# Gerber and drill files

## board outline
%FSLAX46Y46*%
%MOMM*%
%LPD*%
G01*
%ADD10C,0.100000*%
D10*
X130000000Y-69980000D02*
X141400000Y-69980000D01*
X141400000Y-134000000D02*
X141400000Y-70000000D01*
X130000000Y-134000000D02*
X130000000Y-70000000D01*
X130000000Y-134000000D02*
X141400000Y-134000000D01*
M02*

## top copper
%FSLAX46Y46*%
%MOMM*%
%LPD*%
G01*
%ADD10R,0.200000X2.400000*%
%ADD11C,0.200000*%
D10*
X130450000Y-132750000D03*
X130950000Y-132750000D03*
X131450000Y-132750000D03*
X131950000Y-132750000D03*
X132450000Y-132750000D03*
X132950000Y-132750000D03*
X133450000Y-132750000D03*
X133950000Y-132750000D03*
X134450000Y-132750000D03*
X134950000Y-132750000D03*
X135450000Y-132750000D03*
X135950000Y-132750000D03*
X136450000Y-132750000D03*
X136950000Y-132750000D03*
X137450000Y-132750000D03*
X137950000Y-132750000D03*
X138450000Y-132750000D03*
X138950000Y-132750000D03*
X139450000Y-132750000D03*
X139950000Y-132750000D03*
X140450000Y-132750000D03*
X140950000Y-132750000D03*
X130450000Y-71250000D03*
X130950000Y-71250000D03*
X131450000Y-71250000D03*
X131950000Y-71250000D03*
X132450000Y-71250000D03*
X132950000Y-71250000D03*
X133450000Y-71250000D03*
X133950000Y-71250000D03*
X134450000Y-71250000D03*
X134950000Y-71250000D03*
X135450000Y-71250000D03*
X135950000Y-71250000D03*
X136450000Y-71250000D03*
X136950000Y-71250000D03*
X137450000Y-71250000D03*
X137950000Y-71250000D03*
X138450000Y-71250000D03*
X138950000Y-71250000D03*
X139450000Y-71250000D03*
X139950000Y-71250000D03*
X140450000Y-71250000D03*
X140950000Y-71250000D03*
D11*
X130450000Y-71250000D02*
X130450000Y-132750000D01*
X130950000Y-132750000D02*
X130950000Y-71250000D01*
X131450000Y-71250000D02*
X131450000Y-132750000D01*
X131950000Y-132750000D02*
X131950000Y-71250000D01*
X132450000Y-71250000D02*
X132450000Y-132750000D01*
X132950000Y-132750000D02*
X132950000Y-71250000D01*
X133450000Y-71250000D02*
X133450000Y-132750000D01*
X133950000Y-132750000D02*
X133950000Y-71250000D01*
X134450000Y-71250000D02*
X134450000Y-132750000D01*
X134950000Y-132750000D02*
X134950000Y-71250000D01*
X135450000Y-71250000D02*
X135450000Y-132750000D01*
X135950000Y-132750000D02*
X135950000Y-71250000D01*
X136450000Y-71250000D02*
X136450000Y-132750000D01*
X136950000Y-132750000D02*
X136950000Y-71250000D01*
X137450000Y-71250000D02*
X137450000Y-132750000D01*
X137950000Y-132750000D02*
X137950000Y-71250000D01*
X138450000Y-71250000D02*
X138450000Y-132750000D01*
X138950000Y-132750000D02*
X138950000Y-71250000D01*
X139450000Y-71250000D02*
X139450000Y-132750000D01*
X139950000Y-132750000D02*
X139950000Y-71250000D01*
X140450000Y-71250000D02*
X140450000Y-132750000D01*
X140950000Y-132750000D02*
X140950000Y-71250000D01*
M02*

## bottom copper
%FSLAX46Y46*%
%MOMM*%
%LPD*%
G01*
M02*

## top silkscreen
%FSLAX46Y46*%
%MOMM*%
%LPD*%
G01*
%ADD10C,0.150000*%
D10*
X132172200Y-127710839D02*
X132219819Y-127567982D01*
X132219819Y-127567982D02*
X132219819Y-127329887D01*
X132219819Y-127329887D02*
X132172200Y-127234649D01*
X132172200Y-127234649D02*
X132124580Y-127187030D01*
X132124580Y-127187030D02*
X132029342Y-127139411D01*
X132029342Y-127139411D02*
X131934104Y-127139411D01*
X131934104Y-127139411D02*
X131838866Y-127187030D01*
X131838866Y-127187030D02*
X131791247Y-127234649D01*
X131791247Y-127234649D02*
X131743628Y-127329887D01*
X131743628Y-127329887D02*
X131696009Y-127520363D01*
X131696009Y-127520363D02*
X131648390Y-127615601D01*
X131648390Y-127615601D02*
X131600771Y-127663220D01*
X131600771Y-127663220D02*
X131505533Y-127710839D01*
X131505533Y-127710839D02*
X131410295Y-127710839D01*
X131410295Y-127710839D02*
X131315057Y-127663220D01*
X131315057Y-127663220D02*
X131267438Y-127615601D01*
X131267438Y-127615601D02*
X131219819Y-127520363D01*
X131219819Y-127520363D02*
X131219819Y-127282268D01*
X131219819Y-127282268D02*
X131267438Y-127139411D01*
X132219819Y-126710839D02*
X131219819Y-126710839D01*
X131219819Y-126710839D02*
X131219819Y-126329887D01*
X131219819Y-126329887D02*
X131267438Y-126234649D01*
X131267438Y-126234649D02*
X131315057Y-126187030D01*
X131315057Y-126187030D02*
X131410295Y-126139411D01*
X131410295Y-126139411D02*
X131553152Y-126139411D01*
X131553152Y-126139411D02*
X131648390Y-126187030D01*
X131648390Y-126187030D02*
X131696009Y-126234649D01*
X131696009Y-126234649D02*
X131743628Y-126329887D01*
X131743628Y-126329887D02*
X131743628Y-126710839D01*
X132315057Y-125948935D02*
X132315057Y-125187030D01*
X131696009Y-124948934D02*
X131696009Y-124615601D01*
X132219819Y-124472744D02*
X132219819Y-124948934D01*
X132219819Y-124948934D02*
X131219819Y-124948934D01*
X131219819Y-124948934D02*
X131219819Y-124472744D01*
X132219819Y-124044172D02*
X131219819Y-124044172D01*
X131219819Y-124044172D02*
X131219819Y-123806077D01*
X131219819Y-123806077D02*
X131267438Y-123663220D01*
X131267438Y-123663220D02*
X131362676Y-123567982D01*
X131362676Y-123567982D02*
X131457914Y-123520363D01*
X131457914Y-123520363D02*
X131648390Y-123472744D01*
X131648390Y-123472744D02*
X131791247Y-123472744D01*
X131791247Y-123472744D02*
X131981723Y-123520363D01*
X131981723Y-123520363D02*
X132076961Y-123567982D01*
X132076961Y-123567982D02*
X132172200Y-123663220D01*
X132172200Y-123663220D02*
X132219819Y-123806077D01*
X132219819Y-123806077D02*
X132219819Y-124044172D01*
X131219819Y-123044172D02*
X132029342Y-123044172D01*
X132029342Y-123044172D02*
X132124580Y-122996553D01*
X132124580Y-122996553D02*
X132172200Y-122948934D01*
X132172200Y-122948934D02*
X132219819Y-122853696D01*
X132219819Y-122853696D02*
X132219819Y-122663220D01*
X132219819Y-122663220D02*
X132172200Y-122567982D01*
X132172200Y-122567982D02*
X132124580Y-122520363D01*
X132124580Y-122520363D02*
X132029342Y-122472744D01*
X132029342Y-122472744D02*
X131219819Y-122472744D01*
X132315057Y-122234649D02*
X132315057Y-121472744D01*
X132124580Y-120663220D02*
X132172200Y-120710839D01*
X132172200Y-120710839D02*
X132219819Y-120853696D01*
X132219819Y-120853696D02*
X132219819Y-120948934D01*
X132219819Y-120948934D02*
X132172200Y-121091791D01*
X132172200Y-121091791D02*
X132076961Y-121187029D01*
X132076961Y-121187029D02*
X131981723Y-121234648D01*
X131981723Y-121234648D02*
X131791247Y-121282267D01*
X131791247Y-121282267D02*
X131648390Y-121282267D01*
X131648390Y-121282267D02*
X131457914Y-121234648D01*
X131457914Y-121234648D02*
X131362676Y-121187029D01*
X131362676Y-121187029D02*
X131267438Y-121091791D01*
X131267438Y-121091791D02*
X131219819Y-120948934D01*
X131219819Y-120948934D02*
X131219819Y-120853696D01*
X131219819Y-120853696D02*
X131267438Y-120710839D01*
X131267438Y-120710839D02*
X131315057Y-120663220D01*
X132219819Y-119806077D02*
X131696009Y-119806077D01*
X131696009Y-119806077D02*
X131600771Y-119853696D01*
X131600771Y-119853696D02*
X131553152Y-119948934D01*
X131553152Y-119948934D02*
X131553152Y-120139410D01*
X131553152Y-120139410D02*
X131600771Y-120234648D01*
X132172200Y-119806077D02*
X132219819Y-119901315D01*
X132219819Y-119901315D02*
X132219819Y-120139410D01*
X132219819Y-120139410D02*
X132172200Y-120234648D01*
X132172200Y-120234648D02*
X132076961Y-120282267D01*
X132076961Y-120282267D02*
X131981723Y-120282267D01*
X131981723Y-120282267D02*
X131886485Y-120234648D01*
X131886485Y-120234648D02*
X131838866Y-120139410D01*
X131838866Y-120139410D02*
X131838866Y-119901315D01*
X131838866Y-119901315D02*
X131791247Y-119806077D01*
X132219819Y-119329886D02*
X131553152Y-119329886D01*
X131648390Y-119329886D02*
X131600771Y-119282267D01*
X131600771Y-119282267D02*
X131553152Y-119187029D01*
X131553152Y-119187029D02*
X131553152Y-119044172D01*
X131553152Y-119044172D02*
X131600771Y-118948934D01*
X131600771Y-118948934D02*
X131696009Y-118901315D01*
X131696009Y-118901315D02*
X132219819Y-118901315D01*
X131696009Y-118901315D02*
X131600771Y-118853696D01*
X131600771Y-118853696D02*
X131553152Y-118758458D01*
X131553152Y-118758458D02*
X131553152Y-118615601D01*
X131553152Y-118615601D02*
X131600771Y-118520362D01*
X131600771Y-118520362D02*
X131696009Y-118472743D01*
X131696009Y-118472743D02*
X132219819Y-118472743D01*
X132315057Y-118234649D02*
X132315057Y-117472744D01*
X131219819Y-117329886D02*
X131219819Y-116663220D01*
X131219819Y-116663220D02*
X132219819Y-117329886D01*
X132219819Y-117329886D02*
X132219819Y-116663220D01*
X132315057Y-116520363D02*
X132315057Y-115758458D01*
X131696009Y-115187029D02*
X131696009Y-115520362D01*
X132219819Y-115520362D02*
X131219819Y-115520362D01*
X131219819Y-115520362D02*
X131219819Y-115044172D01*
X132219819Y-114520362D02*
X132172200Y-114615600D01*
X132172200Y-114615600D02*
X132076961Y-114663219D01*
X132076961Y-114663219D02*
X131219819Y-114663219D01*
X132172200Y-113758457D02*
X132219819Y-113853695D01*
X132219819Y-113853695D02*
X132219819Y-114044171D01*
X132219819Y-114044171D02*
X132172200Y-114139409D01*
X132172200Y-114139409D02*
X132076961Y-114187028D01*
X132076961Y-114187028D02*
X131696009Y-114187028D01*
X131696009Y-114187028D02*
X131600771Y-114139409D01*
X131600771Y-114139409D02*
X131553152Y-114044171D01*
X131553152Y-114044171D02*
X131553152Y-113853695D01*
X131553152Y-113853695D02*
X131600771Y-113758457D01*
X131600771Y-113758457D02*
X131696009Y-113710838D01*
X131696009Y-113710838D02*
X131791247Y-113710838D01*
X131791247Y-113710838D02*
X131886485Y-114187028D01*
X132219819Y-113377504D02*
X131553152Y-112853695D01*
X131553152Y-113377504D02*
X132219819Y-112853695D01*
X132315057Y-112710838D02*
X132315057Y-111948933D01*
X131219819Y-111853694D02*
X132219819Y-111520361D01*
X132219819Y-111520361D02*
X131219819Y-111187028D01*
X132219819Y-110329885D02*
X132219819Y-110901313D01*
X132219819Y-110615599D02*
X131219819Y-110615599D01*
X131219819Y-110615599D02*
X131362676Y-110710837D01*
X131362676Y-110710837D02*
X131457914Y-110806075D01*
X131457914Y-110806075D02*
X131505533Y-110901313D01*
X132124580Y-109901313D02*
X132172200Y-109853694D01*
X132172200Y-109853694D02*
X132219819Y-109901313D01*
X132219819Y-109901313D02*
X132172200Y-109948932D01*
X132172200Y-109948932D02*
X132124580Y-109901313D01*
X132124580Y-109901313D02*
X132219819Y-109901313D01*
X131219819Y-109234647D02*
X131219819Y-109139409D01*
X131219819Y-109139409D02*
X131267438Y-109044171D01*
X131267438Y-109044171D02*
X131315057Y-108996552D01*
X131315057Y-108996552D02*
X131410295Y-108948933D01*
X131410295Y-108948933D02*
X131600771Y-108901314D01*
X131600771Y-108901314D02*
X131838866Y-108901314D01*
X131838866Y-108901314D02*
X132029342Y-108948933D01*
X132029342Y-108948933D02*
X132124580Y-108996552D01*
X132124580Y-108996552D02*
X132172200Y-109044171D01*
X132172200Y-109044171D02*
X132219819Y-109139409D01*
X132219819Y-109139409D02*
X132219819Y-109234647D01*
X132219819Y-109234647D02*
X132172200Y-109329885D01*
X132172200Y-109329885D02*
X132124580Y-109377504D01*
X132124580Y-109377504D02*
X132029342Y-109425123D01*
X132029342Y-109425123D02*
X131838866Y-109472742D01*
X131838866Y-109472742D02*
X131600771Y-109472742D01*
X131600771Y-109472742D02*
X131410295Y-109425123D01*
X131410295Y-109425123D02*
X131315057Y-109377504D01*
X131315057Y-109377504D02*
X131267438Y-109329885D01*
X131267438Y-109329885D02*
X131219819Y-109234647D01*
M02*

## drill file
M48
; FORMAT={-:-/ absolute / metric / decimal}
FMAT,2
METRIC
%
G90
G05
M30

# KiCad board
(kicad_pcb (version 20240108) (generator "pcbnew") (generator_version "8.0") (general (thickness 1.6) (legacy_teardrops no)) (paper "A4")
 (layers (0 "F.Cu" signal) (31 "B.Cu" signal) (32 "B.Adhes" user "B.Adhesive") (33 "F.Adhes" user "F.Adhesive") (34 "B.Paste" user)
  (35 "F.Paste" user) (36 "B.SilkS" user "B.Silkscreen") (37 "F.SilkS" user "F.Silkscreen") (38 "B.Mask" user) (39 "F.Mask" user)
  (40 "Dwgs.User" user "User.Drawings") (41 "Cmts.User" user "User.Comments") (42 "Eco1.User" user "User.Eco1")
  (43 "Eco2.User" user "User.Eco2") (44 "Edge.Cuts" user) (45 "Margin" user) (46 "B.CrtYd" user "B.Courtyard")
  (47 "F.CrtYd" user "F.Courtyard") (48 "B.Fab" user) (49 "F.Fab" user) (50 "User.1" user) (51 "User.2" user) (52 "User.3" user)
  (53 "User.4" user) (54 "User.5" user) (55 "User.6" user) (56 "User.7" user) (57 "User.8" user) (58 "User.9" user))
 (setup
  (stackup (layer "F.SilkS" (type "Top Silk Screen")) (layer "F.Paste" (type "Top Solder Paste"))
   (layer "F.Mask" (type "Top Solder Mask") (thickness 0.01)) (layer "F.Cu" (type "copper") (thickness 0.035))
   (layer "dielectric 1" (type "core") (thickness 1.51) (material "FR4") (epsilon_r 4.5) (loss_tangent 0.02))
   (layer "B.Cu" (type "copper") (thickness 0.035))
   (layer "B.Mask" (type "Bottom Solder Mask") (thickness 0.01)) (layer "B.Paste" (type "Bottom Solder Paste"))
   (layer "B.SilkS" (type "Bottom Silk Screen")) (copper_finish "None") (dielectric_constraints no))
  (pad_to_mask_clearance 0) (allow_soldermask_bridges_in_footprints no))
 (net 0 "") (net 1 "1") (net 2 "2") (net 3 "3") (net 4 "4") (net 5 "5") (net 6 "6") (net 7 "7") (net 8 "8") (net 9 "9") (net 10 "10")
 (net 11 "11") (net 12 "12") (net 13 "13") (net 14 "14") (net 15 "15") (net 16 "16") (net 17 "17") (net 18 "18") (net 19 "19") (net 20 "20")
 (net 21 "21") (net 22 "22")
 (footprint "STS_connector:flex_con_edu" (layer "F.Cu") (at 130 136.1)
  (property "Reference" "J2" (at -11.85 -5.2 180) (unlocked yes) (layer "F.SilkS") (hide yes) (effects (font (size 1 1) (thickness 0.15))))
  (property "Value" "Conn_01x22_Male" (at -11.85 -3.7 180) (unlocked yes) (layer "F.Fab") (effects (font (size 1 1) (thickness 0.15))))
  (pad "1" smd rect (at 0.45 -3.35) (size 0.2 2.4) (layers "F.Cu" "F.Paste" "F.Mask") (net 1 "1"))
  (pad "2" smd rect (at 0.95 -3.35) (size 0.2 2.4) (layers "F.Cu" "F.Paste" "F.Mask") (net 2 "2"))
  (pad "3" smd rect (at 1.45 -3.35) (size 0.2 2.4) (layers "F.Cu" "F.Paste" "F.Mask") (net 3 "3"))
  (pad "4" smd rect (at 1.95 -3.35) (size 0.2 2.4) (layers "F.Cu" "F.Paste" "F.Mask") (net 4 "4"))
  (pad "5" smd rect (at 2.45 -3.35) (size 0.2 2.4) (layers "F.Cu" "F.Paste" "F.Mask") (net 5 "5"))
  (pad "6" smd rect (at 2.95 -3.35) (size 0.2 2.4) (layers "F.Cu" "F.Paste" "F.Mask") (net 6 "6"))
  (pad "7" smd rect (at 3.45 -3.35) (size 0.2 2.4) (layers "F.Cu" "F.Paste" "F.Mask") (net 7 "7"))
  (pad "8" smd rect (at 3.95 -3.35) (size 0.2 2.4) (layers "F.Cu" "F.Paste" "F.Mask") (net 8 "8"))
  (pad "9" smd rect (at 4.45 -3.35) (size 0.2 2.4) (layers "F.Cu" "F.Paste" "F.Mask") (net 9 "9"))
  (pad "10" smd rect (at 4.95 -3.35) (size 0.2 2.4) (layers "F.Cu" "F.Paste" "F.Mask") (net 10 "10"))
  (pad "11" smd rect (at 5.45 -3.35) (size 0.2 2.4) (layers "F.Cu" "F.Paste" "F.Mask") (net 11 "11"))
  (pad "12" smd rect (at 5.95 -3.35) (size 0.2 2.4) (layers "F.Cu" "F.Paste" "F.Mask") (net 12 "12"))
  (pad "13" smd rect (at 6.45 -3.35) (size 0.2 2.4) (layers "F.Cu" "F.Paste" "F.Mask") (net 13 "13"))
  (pad "14" smd rect (at 6.95 -3.35) (size 0.2 2.4) (layers "F.Cu" "F.Paste" "F.Mask") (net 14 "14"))
  (pad "15" smd rect (at 7.45 -3.35) (size 0.2 2.4) (layers "F.Cu" "F.Paste" "F.Mask") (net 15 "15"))
  (pad "16" smd rect (at 7.95 -3.35) (size 0.2 2.4) (layers "F.Cu" "F.Paste" "F.Mask") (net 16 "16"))
  (pad "17" smd rect (at 8.45 -3.35) (size 0.2 2.4) (layers "F.Cu" "F.Paste" "F.Mask") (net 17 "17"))
  (pad "18" smd rect (at 8.95 -3.35) (size 0.2 2.4) (layers "F.Cu" "F.Paste" "F.Mask") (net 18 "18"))
  (pad "19" smd rect (at 9.45 -3.35) (size 0.2 2.4) (layers "F.Cu" "F.Paste" "F.Mask") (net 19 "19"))
  (pad "20" smd rect (at 9.95 -3.35) (size 0.2 2.4) (layers "F.Cu" "F.Paste" "F.Mask") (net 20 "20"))
  (pad "21" smd rect (at 10.45 -3.35) (size 0.2 2.4) (layers "F.Cu" "F.Paste" "F.Mask") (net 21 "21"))
  (pad "22" smd rect (at 10.95 -3.35) (size 0.2 2.4) (layers "F.Cu" "F.Paste" "F.Mask") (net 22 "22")))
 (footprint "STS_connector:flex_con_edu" (layer "F.Cu") (at 130 74.6)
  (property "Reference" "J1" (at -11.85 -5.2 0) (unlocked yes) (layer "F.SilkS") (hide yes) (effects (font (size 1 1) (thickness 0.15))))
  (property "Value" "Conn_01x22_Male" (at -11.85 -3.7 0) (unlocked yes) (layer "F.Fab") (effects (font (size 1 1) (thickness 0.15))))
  (pad "1" smd rect (at 0.45 -3.35) (size 0.2 2.4) (layers "F.Cu" "F.Paste" "F.Mask") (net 1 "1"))
  (pad "2" smd rect (at 0.95 -3.35) (size 0.2 2.4) (layers "F.Cu" "F.Paste" "F.Mask") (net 2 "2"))
  (pad "3" smd rect (at 1.45 -3.35) (size 0.2 2.4) (layers "F.Cu" "F.Paste" "F.Mask") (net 3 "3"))
  (pad "4" smd rect (at 1.95 -3.35) (size 0.2 2.4) (layers "F.Cu" "F.Paste" "F.Mask") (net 4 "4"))
  (pad "5" smd rect (at 2.45 -3.35) (size 0.2 2.4) (layers "F.Cu" "F.Paste" "F.Mask") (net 5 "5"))
  (pad "6" smd rect (at 2.95 -3.35) (size 0.2 2.4) (layers "F.Cu" "F.Paste" "F.Mask") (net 6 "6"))
  (pad "7" smd rect (at 3.45 -3.35) (size 0.2 2.4) (layers "F.Cu" "F.Paste" "F.Mask") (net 7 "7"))
  (pad "8" smd rect (at 3.95 -3.35) (size 0.2 2.4) (layers "F.Cu" "F.Paste" "F.Mask") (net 8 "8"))
  (pad "9" smd rect (at 4.45 -3.35) (size 0.2 2.4) (layers "F.Cu" "F.Paste" "F.Mask") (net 9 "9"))
  (pad "10" smd rect (at 4.95 -3.35) (size 0.2 2.4) (layers "F.Cu" "F.Paste" "F.Mask") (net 10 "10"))
  (pad "11" smd rect (at 5.45 -3.35) (size 0.2 2.4) (layers "F.Cu" "F.Paste" "F.Mask") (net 11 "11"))
  (pad "12" smd rect (at 5.95 -3.35) (size 0.2 2.4) (layers "F.Cu" "F.Paste" "F.Mask") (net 12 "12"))
  (pad "13" smd rect (at 6.45 -3.35) (size 0.2 2.4) (layers "F.Cu" "F.Paste" "F.Mask") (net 13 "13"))
  (pad "14" smd rect (at 6.95 -3.35) (size 0.2 2.4) (layers "F.Cu" "F.Paste" "F.Mask") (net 14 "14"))
  (pad "15" smd rect (at 7.45 -3.35) (size 0.2 2.4) (layers "F.Cu" "F.Paste" "F.Mask") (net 15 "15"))
  (pad "16" smd rect (at 7.95 -3.35) (size 0.2 2.4) (layers "F.Cu" "F.Paste" "F.Mask") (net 16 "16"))
  (pad "17" smd rect (at 8.45 -3.35) (size 0.2 2.4) (layers "F.Cu" "F.Paste" "F.Mask") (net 17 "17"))
  (pad "18" smd rect (at 8.95 -3.35) (size 0.2 2.4) (layers "F.Cu" "F.Paste" "F.Mask") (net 18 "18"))
  (pad "19" smd rect (at 9.45 -3.35) (size 0.2 2.4) (layers "F.Cu" "F.Paste" "F.Mask") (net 19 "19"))
  (pad "20" smd rect (at 9.95 -3.35) (size 0.2 2.4) (layers "F.Cu" "F.Paste" "F.Mask") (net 20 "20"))
  (pad "21" smd rect (at 10.45 -3.35) (size 0.2 2.4) (layers "F.Cu" "F.Paste" "F.Mask") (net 21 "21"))
  (pad "22" smd rect (at 10.95 -3.35) (size 0.2 2.4) (layers "F.Cu" "F.Paste" "F.Mask") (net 22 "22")))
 (gr_line (start 130 69.98) (end 141.4 69.98) (stroke (width 0.1) (type solid)) (layer "Edge.Cuts"))
 (gr_line (start 141.4 134) (end 141.4 70) (stroke (width 0.1) (type solid)) (layer "Edge.Cuts"))
 (gr_line (start 130 134) (end 130 70) (stroke (width 0.1) (type solid)) (layer "Edge.Cuts"))
 (gr_line (start 130 134) (end 141.4 134) (stroke (width 0.1) (type solid)) (layer "Edge.Cuts"))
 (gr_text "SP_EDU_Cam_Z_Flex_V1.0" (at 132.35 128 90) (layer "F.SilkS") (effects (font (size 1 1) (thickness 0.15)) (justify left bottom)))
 (segment (start 130.45 71.25) (end 130.45 132.75) (width 0.2) (layer "F.Cu") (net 1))
 (segment (start 130.95 132.75) (end 130.95 71.25) (width 0.2) (layer "F.Cu") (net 2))
 (segment (start 131.45 71.25) (end 131.45 132.75) (width 0.2) (layer "F.Cu") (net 3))
 (segment (start 131.95 132.75) (end 131.95 71.25) (width 0.2) (layer "F.Cu") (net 4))
 (segment (start 132.45 71.25) (end 132.45 132.75) (width 0.2) (layer "F.Cu") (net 5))
 (segment (start 132.95 132.75) (end 132.95 71.25) (width 0.2) (layer "F.Cu") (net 6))
 (segment (start 133.45 71.25) (end 133.45 132.75) (width 0.2) (layer "F.Cu") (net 7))
 (segment (start 133.95 132.75) (end 133.95 71.25) (width 0.2) (layer "F.Cu") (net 8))
 (segment (start 134.45 71.25) (end 134.45 132.75) (width 0.2) (layer "F.Cu") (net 9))
 (segment (start 134.95 132.75) (end 134.95 71.25) (width 0.2) (layer "F.Cu") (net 10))
 (segment (start 135.45 71.25) (end 135.45 132.75) (width 0.2) (layer "F.Cu") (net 11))
 (segment (start 135.95 132.75) (end 135.95 71.25) (width 0.2) (layer "F.Cu") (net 12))
 (segment (start 136.45 71.25) (end 136.45 132.75) (width 0.2) (layer "F.Cu") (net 13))
 (segment (start 136.95 132.75) (end 136.95 71.25) (width 0.2) (layer "F.Cu") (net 14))
 (segment (start 137.45 71.25) (end 137.45 132.75) (width 0.2) (layer "F.Cu") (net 15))
 (segment (start 137.95 132.75) (end 137.95 71.25) (width 0.2) (layer "F.Cu") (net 16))
 (segment (start 138.45 71.25) (end 138.45 132.75) (width 0.2) (layer "F.Cu") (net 17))
 (segment (start 138.95 132.75) (end 138.95 71.25) (width 0.2) (layer "F.Cu") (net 18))
 (segment (start 139.45 71.25) (end 139.45 132.75) (width 0.2) (layer "F.Cu") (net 19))
 (segment (start 139.95 132.75) (end 139.95 71.25) (width 0.2) (layer "F.Cu") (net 20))
 (segment (start 140.45 71.25) (end 140.45 132.75) (width 0.2) (layer "F.Cu") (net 21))
 (segment (start 140.95 132.75) (end 140.95 71.25) (width 0.2) (layer "F.Cu") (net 22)))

